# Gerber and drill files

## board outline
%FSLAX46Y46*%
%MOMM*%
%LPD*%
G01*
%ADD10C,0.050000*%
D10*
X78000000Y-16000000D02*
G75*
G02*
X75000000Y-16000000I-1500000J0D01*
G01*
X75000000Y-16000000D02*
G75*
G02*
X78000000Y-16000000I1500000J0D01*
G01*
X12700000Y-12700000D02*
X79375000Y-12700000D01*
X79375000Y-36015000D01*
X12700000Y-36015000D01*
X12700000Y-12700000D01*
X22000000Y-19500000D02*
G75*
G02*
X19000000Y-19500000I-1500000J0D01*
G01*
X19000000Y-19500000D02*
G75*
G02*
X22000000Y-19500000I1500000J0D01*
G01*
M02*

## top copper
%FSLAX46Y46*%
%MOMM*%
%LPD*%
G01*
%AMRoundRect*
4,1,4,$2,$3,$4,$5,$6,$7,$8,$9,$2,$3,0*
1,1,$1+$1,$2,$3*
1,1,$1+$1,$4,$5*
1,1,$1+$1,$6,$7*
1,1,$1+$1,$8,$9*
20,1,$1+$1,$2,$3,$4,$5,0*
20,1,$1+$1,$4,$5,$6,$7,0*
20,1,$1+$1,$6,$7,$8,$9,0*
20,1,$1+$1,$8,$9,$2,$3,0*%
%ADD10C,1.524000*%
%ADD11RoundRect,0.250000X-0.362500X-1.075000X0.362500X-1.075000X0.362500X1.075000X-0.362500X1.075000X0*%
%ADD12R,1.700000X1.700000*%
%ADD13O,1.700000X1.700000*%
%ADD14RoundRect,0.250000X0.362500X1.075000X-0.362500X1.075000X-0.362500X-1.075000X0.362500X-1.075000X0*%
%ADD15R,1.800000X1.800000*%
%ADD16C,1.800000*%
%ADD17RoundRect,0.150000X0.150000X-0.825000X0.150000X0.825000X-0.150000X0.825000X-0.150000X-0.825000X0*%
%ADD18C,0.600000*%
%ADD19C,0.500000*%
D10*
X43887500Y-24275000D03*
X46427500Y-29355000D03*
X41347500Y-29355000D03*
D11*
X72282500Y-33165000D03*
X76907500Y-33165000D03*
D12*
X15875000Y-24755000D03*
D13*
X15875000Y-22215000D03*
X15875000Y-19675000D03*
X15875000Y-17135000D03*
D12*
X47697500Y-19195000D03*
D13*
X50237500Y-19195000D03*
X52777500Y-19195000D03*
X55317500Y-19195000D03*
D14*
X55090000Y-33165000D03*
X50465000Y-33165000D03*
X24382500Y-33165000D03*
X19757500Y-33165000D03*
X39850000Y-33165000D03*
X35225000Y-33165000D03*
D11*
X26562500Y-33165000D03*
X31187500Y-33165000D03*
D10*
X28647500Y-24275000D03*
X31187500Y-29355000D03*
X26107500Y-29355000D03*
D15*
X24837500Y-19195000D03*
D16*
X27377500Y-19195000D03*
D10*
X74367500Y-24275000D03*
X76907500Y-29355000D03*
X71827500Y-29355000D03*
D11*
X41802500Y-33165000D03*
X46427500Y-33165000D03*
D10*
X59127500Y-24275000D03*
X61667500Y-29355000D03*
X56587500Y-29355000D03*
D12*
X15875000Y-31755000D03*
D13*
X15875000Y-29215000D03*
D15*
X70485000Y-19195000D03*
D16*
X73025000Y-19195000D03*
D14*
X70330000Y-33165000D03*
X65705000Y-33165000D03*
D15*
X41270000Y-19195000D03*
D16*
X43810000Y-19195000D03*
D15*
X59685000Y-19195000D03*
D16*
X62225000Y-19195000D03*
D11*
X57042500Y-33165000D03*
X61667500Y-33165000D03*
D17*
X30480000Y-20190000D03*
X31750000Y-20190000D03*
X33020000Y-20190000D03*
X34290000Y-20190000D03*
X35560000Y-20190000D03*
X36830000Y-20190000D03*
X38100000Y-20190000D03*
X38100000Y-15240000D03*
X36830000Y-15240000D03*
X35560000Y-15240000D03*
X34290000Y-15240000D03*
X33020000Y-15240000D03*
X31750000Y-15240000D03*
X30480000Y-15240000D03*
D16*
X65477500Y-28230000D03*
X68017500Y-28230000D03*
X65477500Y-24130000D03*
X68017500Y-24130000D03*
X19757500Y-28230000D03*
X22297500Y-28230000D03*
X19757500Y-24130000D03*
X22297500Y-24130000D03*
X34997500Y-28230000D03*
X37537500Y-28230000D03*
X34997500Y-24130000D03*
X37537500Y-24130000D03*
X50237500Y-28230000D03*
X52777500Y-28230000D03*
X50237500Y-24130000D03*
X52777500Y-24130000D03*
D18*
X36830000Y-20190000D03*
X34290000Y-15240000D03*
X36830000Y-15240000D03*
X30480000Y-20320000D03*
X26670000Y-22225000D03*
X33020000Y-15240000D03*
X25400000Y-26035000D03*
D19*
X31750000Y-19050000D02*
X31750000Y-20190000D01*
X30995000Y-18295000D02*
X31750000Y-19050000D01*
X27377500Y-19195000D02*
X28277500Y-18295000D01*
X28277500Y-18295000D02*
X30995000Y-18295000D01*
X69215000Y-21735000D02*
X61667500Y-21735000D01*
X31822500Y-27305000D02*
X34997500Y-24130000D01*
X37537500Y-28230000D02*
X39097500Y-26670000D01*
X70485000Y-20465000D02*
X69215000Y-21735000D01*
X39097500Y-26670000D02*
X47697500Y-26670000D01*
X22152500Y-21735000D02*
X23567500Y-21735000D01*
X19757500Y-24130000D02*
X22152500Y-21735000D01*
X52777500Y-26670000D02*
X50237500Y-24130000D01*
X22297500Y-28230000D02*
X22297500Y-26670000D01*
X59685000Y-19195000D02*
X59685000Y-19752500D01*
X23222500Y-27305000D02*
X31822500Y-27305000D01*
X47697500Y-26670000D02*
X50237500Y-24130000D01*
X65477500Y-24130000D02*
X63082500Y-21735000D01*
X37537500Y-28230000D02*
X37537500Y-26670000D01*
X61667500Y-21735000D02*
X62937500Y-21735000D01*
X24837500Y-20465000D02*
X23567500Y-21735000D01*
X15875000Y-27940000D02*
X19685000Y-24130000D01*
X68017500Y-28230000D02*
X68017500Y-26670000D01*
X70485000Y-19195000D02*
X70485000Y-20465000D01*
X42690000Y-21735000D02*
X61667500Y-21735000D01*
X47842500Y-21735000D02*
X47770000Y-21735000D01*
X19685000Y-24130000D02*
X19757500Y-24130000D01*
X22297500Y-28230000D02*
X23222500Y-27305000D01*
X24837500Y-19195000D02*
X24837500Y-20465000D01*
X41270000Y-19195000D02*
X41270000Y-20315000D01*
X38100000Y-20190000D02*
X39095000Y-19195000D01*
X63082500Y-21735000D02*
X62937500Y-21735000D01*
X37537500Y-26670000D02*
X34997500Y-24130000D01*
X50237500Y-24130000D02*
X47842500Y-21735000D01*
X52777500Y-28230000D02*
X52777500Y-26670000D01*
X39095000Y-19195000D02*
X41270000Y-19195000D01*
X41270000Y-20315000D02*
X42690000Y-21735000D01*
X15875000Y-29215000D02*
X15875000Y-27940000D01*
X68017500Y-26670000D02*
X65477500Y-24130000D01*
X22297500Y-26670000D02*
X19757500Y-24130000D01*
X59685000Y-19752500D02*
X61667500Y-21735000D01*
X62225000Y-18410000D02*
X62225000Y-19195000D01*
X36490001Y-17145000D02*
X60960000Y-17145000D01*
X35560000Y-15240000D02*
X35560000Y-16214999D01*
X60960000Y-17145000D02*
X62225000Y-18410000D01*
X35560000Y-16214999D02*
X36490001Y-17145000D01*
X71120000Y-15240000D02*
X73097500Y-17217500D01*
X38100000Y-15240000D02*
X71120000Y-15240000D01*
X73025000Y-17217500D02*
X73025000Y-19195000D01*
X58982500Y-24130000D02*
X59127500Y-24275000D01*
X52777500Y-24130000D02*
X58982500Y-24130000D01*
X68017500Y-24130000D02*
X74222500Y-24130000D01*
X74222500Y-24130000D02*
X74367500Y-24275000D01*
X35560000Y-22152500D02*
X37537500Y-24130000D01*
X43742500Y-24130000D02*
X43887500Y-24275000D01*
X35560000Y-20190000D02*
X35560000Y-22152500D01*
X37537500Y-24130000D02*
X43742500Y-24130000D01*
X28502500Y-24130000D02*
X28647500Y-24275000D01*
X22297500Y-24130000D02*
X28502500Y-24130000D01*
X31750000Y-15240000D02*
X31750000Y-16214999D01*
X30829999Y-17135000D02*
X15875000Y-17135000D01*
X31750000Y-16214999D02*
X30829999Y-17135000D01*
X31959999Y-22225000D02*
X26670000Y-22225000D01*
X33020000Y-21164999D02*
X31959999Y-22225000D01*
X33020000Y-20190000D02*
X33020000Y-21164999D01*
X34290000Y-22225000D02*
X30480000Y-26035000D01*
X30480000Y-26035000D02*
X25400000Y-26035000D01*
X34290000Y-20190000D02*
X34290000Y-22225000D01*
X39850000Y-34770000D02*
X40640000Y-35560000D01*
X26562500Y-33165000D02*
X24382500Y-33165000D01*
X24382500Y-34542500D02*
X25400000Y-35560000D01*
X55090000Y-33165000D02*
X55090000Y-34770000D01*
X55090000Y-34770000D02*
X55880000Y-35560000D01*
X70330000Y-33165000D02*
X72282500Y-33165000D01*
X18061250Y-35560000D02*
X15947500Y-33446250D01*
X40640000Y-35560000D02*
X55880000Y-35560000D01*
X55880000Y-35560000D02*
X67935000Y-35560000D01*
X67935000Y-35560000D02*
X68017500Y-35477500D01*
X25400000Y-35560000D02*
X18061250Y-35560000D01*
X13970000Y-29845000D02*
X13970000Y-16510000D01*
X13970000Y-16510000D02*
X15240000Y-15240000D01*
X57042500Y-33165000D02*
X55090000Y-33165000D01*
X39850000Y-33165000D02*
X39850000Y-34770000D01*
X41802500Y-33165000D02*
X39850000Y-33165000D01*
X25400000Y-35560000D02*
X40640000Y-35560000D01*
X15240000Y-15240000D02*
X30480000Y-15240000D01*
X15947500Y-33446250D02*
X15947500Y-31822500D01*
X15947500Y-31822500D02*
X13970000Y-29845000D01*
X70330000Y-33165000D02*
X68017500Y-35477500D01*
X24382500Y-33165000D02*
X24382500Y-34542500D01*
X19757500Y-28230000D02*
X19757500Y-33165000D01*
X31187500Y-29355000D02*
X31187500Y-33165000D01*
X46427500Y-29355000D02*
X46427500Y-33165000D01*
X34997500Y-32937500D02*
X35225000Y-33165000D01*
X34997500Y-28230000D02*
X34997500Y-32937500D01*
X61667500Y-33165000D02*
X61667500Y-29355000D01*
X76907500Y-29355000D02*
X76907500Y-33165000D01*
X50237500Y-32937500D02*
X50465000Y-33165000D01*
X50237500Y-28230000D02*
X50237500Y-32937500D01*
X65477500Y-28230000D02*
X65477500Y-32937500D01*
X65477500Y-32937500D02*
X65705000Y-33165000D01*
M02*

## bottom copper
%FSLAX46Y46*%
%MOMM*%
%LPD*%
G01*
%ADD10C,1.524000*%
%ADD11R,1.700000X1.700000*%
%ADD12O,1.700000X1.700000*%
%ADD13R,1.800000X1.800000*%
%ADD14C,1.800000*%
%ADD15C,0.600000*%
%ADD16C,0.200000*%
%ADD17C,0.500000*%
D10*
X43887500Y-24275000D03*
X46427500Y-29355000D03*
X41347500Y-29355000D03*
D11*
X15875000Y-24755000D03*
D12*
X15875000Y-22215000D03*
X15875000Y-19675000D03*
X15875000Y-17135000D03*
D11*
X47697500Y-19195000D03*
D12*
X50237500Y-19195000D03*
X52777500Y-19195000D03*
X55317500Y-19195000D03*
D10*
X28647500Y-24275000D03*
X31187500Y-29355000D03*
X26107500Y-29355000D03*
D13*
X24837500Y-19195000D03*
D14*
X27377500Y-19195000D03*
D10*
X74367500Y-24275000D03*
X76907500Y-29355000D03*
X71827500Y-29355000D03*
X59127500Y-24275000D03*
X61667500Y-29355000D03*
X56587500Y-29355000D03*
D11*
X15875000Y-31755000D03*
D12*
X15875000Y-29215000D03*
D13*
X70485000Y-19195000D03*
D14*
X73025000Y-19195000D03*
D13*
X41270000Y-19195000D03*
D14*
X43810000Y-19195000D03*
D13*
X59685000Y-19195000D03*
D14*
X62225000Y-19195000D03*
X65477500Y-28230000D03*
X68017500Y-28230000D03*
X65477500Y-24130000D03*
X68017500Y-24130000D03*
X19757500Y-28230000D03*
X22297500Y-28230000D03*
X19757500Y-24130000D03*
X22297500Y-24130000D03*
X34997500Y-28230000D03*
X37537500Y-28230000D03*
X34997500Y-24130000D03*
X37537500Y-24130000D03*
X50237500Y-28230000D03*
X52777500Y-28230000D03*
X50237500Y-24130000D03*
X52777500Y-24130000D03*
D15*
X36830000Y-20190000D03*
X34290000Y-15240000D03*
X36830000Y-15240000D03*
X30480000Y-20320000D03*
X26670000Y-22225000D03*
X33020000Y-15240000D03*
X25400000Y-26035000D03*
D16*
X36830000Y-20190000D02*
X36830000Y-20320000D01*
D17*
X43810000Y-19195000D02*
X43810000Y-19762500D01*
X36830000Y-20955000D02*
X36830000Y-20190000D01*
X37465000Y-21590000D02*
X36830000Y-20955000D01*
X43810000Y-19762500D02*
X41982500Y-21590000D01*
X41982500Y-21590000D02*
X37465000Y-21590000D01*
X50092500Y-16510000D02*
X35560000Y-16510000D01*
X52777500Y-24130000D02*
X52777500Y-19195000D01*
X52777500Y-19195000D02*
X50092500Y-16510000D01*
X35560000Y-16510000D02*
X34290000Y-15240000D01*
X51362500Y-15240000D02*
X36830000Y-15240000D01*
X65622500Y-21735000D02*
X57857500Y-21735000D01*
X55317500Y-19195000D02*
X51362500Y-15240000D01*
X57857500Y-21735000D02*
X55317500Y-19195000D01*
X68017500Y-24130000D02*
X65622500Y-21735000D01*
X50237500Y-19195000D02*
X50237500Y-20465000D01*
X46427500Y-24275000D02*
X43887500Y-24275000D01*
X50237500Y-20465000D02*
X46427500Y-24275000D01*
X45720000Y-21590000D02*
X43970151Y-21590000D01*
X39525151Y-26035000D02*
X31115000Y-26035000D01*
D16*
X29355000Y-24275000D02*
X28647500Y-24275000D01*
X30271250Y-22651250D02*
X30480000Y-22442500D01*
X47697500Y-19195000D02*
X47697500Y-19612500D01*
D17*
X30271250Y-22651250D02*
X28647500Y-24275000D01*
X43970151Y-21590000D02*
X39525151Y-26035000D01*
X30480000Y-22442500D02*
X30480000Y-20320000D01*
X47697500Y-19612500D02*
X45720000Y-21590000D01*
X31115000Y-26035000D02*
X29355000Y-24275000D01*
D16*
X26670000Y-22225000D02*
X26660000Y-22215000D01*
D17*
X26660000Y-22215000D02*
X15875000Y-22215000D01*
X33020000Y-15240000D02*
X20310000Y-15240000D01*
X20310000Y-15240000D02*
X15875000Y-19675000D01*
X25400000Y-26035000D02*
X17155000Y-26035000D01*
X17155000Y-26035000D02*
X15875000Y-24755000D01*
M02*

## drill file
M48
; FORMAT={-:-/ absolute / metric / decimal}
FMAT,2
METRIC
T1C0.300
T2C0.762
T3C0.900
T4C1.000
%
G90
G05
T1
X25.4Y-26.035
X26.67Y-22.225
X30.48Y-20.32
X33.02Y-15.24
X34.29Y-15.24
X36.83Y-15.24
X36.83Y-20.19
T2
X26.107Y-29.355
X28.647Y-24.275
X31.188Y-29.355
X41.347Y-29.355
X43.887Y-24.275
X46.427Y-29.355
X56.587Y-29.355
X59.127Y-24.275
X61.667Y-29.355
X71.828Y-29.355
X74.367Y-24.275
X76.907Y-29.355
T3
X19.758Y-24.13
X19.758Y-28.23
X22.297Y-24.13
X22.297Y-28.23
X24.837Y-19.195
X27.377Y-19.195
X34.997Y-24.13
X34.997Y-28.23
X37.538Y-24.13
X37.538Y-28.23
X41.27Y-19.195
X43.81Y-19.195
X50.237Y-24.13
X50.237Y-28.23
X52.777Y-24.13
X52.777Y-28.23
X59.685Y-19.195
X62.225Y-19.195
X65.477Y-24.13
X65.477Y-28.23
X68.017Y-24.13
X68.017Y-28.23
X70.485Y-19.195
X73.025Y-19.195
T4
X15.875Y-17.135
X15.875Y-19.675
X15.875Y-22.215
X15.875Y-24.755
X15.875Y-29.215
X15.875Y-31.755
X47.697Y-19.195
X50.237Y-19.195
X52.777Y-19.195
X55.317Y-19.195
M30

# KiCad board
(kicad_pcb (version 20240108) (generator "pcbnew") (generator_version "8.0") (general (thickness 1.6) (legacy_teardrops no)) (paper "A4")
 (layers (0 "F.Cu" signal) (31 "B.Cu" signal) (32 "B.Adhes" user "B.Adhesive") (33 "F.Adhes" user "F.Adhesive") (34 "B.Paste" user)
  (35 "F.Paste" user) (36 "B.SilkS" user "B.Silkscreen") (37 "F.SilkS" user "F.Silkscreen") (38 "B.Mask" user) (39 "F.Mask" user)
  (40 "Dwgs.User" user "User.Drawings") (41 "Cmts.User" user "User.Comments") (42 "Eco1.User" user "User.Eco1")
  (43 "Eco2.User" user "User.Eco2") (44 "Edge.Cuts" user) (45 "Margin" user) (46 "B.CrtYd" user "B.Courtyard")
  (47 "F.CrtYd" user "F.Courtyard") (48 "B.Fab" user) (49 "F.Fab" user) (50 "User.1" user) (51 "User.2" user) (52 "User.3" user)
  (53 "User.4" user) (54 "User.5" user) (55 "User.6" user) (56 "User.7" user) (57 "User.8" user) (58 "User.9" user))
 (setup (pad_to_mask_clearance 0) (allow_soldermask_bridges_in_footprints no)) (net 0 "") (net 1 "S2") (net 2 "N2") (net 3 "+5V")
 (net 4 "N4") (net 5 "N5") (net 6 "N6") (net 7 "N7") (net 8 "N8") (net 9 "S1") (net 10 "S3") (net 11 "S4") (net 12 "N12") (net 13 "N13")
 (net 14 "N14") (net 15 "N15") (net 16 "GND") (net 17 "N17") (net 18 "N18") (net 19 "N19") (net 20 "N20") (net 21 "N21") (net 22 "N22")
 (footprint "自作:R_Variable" (layer "F.Cu") (at 43.8875 26.815)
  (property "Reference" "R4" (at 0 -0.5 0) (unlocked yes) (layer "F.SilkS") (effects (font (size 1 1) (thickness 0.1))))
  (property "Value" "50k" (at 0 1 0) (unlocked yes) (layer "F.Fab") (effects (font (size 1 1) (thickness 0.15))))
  (pad "1" thru_hole circle (at 0 -2.54) (size 1.524 1.524) (drill 0.762) (layers "*.Cu" "*.Mask") (remove_unused_layers no) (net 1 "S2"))
  (pad "2" thru_hole circle (at 2.54 2.54) (size 1.524 1.524) (drill 0.762) (layers "*.Cu" "*.Mask") (remove_unused_layers no) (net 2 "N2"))
  (pad "3" thru_hole circle (at -2.54 2.54) (size 1.524 1.524) (drill 0.762) (layers "*.Cu" "*.Mask") (remove_unused_layers no)))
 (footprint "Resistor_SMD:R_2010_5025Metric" (layer "F.Cu") (at 74.595 33.165)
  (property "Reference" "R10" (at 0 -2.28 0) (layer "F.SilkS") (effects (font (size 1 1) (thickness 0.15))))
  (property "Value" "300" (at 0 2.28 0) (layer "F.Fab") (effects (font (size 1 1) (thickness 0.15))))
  (pad "1" smd roundrect (at -2.3125 0) (size 1.225 2.65) (layers "F.Cu" "F.Paste" "F.Mask") (roundrect_rratio 0.204082) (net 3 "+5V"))
  (pad "2" smd roundrect (at 2.3125 0) (size 1.225 2.65) (layers "F.Cu" "F.Paste" "F.Mask") (roundrect_rratio 0.204082) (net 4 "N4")))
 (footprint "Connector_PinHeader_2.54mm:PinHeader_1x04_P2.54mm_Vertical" (layer "F.Cu") (at 15.875 24.755 180)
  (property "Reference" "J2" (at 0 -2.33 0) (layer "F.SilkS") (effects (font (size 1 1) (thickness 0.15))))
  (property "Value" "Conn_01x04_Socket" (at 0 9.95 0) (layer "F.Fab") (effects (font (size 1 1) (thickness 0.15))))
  (pad "1" thru_hole rect (at 0 0 180) (size 1.7 1.7) (drill 1) (layers "*.Cu" "*.Mask") (remove_unused_layers no) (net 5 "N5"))
  (pad "2" thru_hole oval (at 0 2.54 180) (size 1.7 1.7) (drill 1) (layers "*.Cu" "*.Mask") (remove_unused_layers no) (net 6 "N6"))
  (pad "3" thru_hole oval (at 0 5.08 180) (size 1.7 1.7) (drill 1) (layers "*.Cu" "*.Mask") (remove_unused_layers no) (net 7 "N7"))
  (pad "4" thru_hole oval (at 0 7.62 180) (size 1.7 1.7) (drill 1) (layers "*.Cu" "*.Mask") (remove_unused_layers no) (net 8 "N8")))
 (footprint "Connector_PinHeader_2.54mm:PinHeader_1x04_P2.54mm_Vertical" (layer "F.Cu") (at 47.6975 19.195 90)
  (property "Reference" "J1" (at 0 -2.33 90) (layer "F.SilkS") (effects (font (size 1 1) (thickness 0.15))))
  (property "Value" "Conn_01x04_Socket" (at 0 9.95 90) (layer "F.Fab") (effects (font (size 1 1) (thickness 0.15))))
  (pad "1" thru_hole rect (at 0 0 90) (size 1.7 1.7) (drill 1) (layers "*.Cu" "*.Mask") (remove_unused_layers no) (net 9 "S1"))
  (pad "2" thru_hole oval (at 0 2.54 90) (size 1.7 1.7) (drill 1) (layers "*.Cu" "*.Mask") (remove_unused_layers no) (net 1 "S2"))
  (pad "3" thru_hole oval (at 0 5.08 90) (size 1.7 1.7) (drill 1) (layers "*.Cu" "*.Mask") (remove_unused_layers no) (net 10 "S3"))
  (pad "4" thru_hole oval (at 0 7.62 90) (size 1.7 1.7) (drill 1) (layers "*.Cu" "*.Mask") (remove_unused_layers no) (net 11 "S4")))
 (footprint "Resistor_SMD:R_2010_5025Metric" (layer "F.Cu") (at 52.7775 33.165 180)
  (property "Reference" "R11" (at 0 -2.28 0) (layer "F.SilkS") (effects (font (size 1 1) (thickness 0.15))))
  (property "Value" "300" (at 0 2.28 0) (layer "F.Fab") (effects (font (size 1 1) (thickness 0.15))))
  (pad "1" smd roundrect (at -2.3125 0 180) (size 1.225 2.65) (layers "F.Cu" "F.Paste" "F.Mask") (roundrect_rratio 0.204082) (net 3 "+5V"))
  (pad "2" smd roundrect (at 2.3125 0 180) (size 1.225 2.65) (layers "F.Cu" "F.Paste" "F.Mask") (roundrect_rratio 0.204082) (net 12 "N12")))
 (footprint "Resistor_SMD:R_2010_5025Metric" (layer "F.Cu") (at 22.07 33.165 180)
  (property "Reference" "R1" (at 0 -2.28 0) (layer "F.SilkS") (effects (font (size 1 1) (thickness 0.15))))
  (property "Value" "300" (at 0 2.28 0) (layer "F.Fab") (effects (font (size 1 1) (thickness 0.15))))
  (pad "1" smd roundrect (at -2.3125 0 180) (size 1.225 2.65) (layers "F.Cu" "F.Paste" "F.Mask") (roundrect_rratio 0.204082) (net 3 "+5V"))
  (pad "2" smd roundrect (at 2.3125 0 180) (size 1.225 2.65) (layers "F.Cu" "F.Paste" "F.Mask") (roundrect_rratio 0.204082) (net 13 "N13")))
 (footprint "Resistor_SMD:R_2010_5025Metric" (layer "F.Cu") (at 37.5375 33.165 180)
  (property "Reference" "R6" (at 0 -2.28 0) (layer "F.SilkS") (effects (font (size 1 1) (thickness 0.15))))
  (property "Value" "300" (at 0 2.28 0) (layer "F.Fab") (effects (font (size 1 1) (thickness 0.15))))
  (pad "1" smd roundrect (at -2.3125 0 180) (size 1.225 2.65) (layers "F.Cu" "F.Paste" "F.Mask") (roundrect_rratio 0.204082) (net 3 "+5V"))
  (pad "2" smd roundrect (at 2.3125 0 180) (size 1.225 2.65) (layers "F.Cu" "F.Paste" "F.Mask") (roundrect_rratio 0.204082) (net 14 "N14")))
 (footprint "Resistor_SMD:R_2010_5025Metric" (layer "F.Cu") (at 28.875 33.165)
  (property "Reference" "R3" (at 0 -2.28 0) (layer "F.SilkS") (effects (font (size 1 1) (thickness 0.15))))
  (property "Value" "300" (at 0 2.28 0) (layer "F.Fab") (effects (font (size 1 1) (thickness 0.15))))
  (pad "1" smd roundrect (at -2.3125 0) (size 1.225 2.65) (layers "F.Cu" "F.Paste" "F.Mask") (roundrect_rratio 0.204082) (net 3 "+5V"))
  (pad "2" smd roundrect (at 2.3125 0) (size 1.225 2.65) (layers "F.Cu" "F.Paste" "F.Mask") (roundrect_rratio 0.204082) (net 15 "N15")))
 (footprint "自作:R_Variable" (layer "F.Cu") (at 28.6475 26.815)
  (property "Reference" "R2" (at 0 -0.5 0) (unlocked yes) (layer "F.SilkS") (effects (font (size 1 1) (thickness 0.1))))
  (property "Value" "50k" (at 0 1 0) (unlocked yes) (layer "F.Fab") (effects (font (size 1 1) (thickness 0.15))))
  (pad "1" thru_hole circle (at 0 -2.54) (size 1.524 1.524) (drill 0.762) (layers "*.Cu" "*.Mask") (remove_unused_layers no) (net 9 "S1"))
  (pad "2" thru_hole circle (at 2.54 2.54) (size 1.524 1.524) (drill 0.762) (layers "*.Cu" "*.Mask") (remove_unused_layers no)
   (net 15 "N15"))
  (pad "3" thru_hole circle (at -2.54 2.54) (size 1.524 1.524) (drill 0.762) (layers "*.Cu" "*.Mask") (remove_unused_layers no)))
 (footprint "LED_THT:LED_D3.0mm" (layer "F.Cu") (at 24.8375 19.195)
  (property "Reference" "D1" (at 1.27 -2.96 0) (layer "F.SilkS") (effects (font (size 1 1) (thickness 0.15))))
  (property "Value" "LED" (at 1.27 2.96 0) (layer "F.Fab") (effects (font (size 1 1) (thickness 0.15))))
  (pad "1" thru_hole rect (at 0 0) (size 1.8 1.8) (drill 0.9) (layers "*.Cu" "*.Mask") (remove_unused_layers no) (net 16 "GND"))
  (pad "2" thru_hole circle (at 2.54 0) (size 1.8 1.8) (drill 0.9) (layers "*.Cu" "*.Mask") (remove_unused_layers no) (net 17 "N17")))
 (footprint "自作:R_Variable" (layer "F.Cu") (at 74.3675 26.815)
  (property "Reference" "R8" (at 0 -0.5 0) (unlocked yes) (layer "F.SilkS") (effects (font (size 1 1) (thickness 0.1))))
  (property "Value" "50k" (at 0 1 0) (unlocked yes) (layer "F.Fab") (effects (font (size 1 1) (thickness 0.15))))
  (pad "1" thru_hole circle (at 0 -2.54) (size 1.524 1.524) (drill 0.762) (layers "*.Cu" "*.Mask") (remove_unused_layers no) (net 11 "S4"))
  (pad "2" thru_hole circle (at 2.54 2.54) (size 1.524 1.524) (drill 0.762) (layers "*.Cu" "*.Mask") (remove_unused_layers no) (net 4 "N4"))
  (pad "3" thru_hole circle (at -2.54 2.54) (size 1.524 1.524) (drill 0.762) (layers "*.Cu" "*.Mask") (remove_unused_layers no)))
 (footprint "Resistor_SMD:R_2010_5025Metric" (layer "F.Cu") (at 44.115 33.165)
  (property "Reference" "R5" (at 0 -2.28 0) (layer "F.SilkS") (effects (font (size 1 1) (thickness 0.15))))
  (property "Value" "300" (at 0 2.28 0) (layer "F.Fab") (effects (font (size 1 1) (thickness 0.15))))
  (pad "1" smd roundrect (at -2.3125 0) (size 1.225 2.65) (layers "F.Cu" "F.Paste" "F.Mask") (roundrect_rratio 0.204082) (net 3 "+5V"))
  (pad "2" smd roundrect (at 2.3125 0) (size 1.225 2.65) (layers "F.Cu" "F.Paste" "F.Mask") (roundrect_rratio 0.204082) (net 2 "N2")))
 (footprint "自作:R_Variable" (layer "F.Cu") (at 59.1275 26.815)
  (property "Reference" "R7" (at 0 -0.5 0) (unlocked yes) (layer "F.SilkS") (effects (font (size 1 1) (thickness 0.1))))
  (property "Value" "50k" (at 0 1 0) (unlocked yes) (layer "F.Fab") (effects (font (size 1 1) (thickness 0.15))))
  (pad "1" thru_hole circle (at 0 -2.54) (size 1.524 1.524) (drill 0.762) (layers "*.Cu" "*.Mask") (remove_unused_layers no) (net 10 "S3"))
  (pad "2" thru_hole circle (at 2.54 2.54) (size 1.524 1.524) (drill 0.762) (layers "*.Cu" "*.Mask") (remove_unused_layers no)
   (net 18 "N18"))
  (pad "3" thru_hole circle (at -2.54 2.54) (size 1.524 1.524) (drill 0.762) (layers "*.Cu" "*.Mask") (remove_unused_layers no)))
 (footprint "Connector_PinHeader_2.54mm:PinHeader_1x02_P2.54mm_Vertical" (layer "F.Cu") (at 15.875 31.755 180)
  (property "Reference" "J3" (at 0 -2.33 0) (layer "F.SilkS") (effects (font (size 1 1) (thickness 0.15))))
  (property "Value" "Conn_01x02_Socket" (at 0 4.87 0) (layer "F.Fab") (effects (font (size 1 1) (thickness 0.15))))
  (pad "1" thru_hole rect (at 0 0 180) (size 1.7 1.7) (drill 1) (layers "*.Cu" "*.Mask") (remove_unused_layers no) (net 3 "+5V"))
  (pad "2" thru_hole oval (at 0 2.54 180) (size 1.7 1.7) (drill 1) (layers "*.Cu" "*.Mask") (remove_unused_layers no) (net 16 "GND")))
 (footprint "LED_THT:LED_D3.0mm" (layer "F.Cu") (at 70.485 19.195)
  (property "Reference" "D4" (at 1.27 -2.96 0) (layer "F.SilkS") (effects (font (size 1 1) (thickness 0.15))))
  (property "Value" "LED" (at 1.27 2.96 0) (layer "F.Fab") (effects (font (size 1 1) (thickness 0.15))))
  (pad "1" thru_hole rect (at 0 0) (size 1.8 1.8) (drill 0.9) (layers "*.Cu" "*.Mask") (remove_unused_layers no) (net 16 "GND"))
  (pad "2" thru_hole circle (at 2.54 0) (size 1.8 1.8) (drill 0.9) (layers "*.Cu" "*.Mask") (remove_unused_layers no) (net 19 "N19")))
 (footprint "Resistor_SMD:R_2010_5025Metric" (layer "F.Cu") (at 68.0175 33.165 180)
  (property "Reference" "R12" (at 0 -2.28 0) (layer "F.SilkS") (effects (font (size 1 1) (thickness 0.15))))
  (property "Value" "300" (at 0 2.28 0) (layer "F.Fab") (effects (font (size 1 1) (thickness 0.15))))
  (pad "1" smd roundrect (at -2.3125 0 180) (size 1.225 2.65) (layers "F.Cu" "F.Paste" "F.Mask") (roundrect_rratio 0.204082) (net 3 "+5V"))
  (pad "2" smd roundrect (at 2.3125 0 180) (size 1.225 2.65) (layers "F.Cu" "F.Paste" "F.Mask") (roundrect_rratio 0.204082) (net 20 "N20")))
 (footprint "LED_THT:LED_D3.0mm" (layer "F.Cu") (at 41.27 19.195)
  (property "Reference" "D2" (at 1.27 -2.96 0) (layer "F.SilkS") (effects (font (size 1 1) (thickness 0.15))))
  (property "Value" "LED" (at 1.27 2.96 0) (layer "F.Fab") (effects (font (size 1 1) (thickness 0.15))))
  (pad "1" thru_hole rect (at 0 0) (size 1.8 1.8) (drill 0.9) (layers "*.Cu" "*.Mask") (remove_unused_layers no) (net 16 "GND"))
  (pad "2" thru_hole circle (at 2.54 0) (size 1.8 1.8) (drill 0.9) (layers "*.Cu" "*.Mask") (remove_unused_layers no) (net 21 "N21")))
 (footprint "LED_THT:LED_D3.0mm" (layer "F.Cu") (at 59.685 19.195)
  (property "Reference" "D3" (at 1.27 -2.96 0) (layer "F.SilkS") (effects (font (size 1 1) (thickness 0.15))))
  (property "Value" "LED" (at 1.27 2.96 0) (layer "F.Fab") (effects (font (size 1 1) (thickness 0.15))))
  (pad "1" thru_hole rect (at 0 0) (size 1.8 1.8) (drill 0.9) (layers "*.Cu" "*.Mask") (remove_unused_layers no) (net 16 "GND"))
  (pad "2" thru_hole circle (at 2.54 0) (size 1.8 1.8) (drill 0.9) (layers "*.Cu" "*.Mask") (remove_unused_layers no) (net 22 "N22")))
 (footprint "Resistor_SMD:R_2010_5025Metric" (layer "F.Cu") (at 59.355 33.165)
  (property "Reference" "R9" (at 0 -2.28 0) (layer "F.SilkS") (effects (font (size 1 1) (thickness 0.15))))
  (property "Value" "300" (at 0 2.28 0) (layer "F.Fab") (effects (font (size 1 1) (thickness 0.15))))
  (pad "1" smd roundrect (at -2.3125 0) (size 1.225 2.65) (layers "F.Cu" "F.Paste" "F.Mask") (roundrect_rratio 0.204082) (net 3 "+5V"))
  (pad "2" smd roundrect (at 2.3125 0) (size 1.225 2.65) (layers "F.Cu" "F.Paste" "F.Mask") (roundrect_rratio 0.204082) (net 18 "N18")))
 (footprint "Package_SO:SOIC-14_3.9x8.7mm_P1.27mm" (layer "F.Cu") (at 34.29 17.715 90)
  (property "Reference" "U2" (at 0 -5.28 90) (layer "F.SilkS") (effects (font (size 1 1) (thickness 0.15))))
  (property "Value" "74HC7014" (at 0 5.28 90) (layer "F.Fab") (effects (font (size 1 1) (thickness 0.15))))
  (pad "1" smd roundrect (at -2.475 -3.81 90) (size 1.95 0.6) (layers "F.Cu" "F.Paste" "F.Mask") (roundrect_rratio 0.25) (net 9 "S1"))
  (pad "2" smd roundrect (at -2.475 -2.54 90) (size 1.95 0.6) (layers "F.Cu" "F.Paste" "F.Mask") (roundrect_rratio 0.25) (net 17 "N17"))
  (pad "3" smd roundrect (at -2.475 -1.27 90) (size 1.95 0.6) (layers "F.Cu" "F.Paste" "F.Mask") (roundrect_rratio 0.25) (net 6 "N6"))
  (pad "4" smd roundrect (at -2.475 0 90) (size 1.95 0.6) (layers "F.Cu" "F.Paste" "F.Mask") (roundrect_rratio 0.25) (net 5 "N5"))
  (pad "5" smd roundrect (at -2.475 1.27 90) (size 1.95 0.6) (layers "F.Cu" "F.Paste" "F.Mask") (roundrect_rratio 0.25) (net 1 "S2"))
  (pad "6" smd roundrect (at -2.475 2.54 90) (size 1.95 0.6) (layers "F.Cu" "F.Paste" "F.Mask") (roundrect_rratio 0.25) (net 21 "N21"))
  (pad "7" smd roundrect (at -2.475 3.81 90) (size 1.95 0.6) (layers "F.Cu" "F.Paste" "F.Mask") (roundrect_rratio 0.25) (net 16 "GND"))
  (pad "8" smd roundrect (at 2.475 3.81 90) (size 1.95 0.6) (layers "F.Cu" "F.Paste" "F.Mask") (roundrect_rratio 0.25) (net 19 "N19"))
  (pad "9" smd roundrect (at 2.475 2.54 90) (size 1.95 0.6) (layers "F.Cu" "F.Paste" "F.Mask") (roundrect_rratio 0.25) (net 11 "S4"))
  (pad "10" smd roundrect (at 2.475 1.27 90) (size 1.95 0.6) (layers "F.Cu" "F.Paste" "F.Mask") (roundrect_rratio 0.25) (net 22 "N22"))
  (pad "11" smd roundrect (at 2.475 0 90) (size 1.95 0.6) (layers "F.Cu" "F.Paste" "F.Mask") (roundrect_rratio 0.25) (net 10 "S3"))
  (pad "12" smd roundrect (at 2.475 -1.27 90) (size 1.95 0.6) (layers "F.Cu" "F.Paste" "F.Mask") (roundrect_rratio 0.25) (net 7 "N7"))
  (pad "13" smd roundrect (at 2.475 -2.54 90) (size 1.95 0.6) (layers "F.Cu" "F.Paste" "F.Mask") (roundrect_rratio 0.25) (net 8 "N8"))
  (pad "14" smd roundrect (at 2.475 -3.81 90) (size 1.95 0.6) (layers "F.Cu" "F.Paste" "F.Mask") (roundrect_rratio 0.25) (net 3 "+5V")))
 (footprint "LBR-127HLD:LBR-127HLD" (layer "B.Cu") (at 66.7475 26.18 -90)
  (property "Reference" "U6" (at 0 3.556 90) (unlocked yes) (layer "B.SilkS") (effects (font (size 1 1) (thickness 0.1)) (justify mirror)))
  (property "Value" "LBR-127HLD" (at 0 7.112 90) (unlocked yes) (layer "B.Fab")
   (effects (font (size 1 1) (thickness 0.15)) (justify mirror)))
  (pad "1" thru_hole circle (at 2.05 1.27 270) (size 1.8 1.8) (drill 0.9) (layers "*.Cu" "*.Mask") (remove_unused_layers no) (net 20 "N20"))
  (pad "2" thru_hole circle (at 2.05 -1.27 270) (size 1.8 1.8) (drill 0.9) (layers "*.Cu" "*.Mask") (remove_unused_layers no) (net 16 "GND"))
  (pad "3" thru_hole circle (at -2.05 1.27 270) (size 1.8 1.8) (drill 0.9) (layers "*.Cu" "*.Mask") (remove_unused_layers no) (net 16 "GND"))
  (pad "4" thru_hole circle (at -2.05 -1.27 270) (size 1.8 1.8) (drill 0.9) (layers "*.Cu" "*.Mask") (remove_unused_layers no) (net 11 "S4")))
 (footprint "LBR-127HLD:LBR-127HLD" (layer "B.Cu") (at 21.0275 26.18 -90)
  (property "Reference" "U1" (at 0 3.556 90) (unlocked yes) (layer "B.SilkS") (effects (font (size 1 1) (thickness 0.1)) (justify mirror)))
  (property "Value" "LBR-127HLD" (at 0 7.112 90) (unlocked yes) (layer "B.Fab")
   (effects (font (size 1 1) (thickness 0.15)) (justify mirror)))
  (pad "1" thru_hole circle (at 2.05 1.27 270) (size 1.8 1.8) (drill 0.9) (layers "*.Cu" "*.Mask") (remove_unused_layers no) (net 13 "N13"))
  (pad "2" thru_hole circle (at 2.05 -1.27 270) (size 1.8 1.8) (drill 0.9) (layers "*.Cu" "*.Mask") (remove_unused_layers no) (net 16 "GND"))
  (pad "3" thru_hole circle (at -2.05 1.27 270) (size 1.8 1.8) (drill 0.9) (layers "*.Cu" "*.Mask") (remove_unused_layers no) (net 16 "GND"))
  (pad "4" thru_hole circle (at -2.05 -1.27 270) (size 1.8 1.8) (drill 0.9) (layers "*.Cu" "*.Mask") (remove_unused_layers no) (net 9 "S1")))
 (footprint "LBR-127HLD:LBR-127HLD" (layer "B.Cu") (at 36.2675 26.18 -90)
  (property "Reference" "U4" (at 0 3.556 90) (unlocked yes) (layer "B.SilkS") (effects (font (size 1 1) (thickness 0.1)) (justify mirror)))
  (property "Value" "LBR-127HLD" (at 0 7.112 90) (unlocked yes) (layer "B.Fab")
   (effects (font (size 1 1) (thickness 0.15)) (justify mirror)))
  (pad "1" thru_hole circle (at 2.05 1.27 270) (size 1.8 1.8) (drill 0.9) (layers "*.Cu" "*.Mask") (remove_unused_layers no) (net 14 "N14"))
  (pad "2" thru_hole circle (at 2.05 -1.27 270) (size 1.8 1.8) (drill 0.9) (layers "*.Cu" "*.Mask") (remove_unused_layers no) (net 16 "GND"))
  (pad "3" thru_hole circle (at -2.05 1.27 270) (size 1.8 1.8) (drill 0.9) (layers "*.Cu" "*.Mask") (remove_unused_layers no) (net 16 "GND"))
  (pad "4" thru_hole circle (at -2.05 -1.27 270) (size 1.8 1.8) (drill 0.9) (layers "*.Cu" "*.Mask") (remove_unused_layers no) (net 1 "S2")))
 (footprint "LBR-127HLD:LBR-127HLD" (layer "B.Cu") (at 51.5075 26.18 -90)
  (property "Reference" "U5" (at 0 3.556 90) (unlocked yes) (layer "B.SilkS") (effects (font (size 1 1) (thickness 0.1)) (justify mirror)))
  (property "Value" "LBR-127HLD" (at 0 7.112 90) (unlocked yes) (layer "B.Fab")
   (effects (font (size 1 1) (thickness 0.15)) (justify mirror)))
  (pad "1" thru_hole circle (at 2.05 1.27 270) (size 1.8 1.8) (drill 0.9) (layers "*.Cu" "*.Mask") (remove_unused_layers no) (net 12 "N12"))
  (pad "2" thru_hole circle (at 2.05 -1.27 270) (size 1.8 1.8) (drill 0.9) (layers "*.Cu" "*.Mask") (remove_unused_layers no) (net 16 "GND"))
  (pad "3" thru_hole circle (at -2.05 1.27 270) (size 1.8 1.8) (drill 0.9) (layers "*.Cu" "*.Mask") (remove_unused_layers no) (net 16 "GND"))
  (pad "4" thru_hole circle (at -2.05 -1.27 270) (size 1.8 1.8) (drill 0.9) (layers "*.Cu" "*.Mask") (remove_unused_layers no) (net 10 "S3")))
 (gr_circle (center 76.5 16) (end 78 16) (stroke (width 0.05) (type default)) (fill none) (layer "Edge.Cuts"))
 (gr_rect (start 12.7 12.7) (end 79.375 36.015) (stroke (width 0.05) (type default)) (fill none) (layer "Edge.Cuts"))
 (gr_circle (center 20.5 19.5) (end 22 19.5) (stroke (width 0.05) (type default)) (fill none) (layer "Edge.Cuts"))
 (segment (start 31.75 19.05) (end 31.75 20.19) (width 0.5) (layer "F.Cu") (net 17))
 (segment (start 30.995 18.295) (end 31.75 19.05) (width 0.5) (layer "F.Cu") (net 17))
 (segment (start 27.3775 19.195) (end 28.2775 18.295) (width 0.5) (layer "F.Cu") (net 17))
 (segment (start 28.2775 18.295) (end 30.995 18.295) (width 0.5) (layer "F.Cu") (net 17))
 (segment (start 69.215 21.735) (end 61.6675 21.735) (width 0.5) (layer "F.Cu") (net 16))
 (segment (start 31.8225 27.305) (end 34.9975 24.13) (width 0.5) (layer "F.Cu") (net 16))
 (segment (start 37.5375 28.23) (end 39.0975 26.67) (width 0.5) (layer "F.Cu") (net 16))
 (segment (start 70.485 20.465) (end 69.215 21.735) (width 0.5) (layer "F.Cu") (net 16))
 (segment (start 39.0975 26.67) (end 47.6975 26.67) (width 0.5) (layer "F.Cu") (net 16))
 (segment (start 22.1525 21.735) (end 23.5675 21.735) (width 0.5) (layer "F.Cu") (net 16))
 (segment (start 19.7575 24.13) (end 22.1525 21.735) (width 0.5) (layer "F.Cu") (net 16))
 (segment (start 52.7775 26.67) (end 50.2375 24.13) (width 0.5) (layer "F.Cu") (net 16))
 (segment (start 22.2975 28.23) (end 22.2975 26.67) (width 0.5) (layer "F.Cu") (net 16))
 (segment (start 59.685 19.195) (end 59.685 19.7525) (width 0.5) (layer "F.Cu") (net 16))
 (segment (start 23.2225 27.305) (end 31.8225 27.305) (width 0.5) (layer "F.Cu") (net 16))
 (segment (start 47.6975 26.67) (end 50.2375 24.13) (width 0.5) (layer "F.Cu") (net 16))
 (segment (start 65.4775 24.13) (end 63.0825 21.735) (width 0.5) (layer "F.Cu") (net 16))
 (segment (start 37.5375 28.23) (end 37.5375 26.67) (width 0.5) (layer "F.Cu") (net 16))
 (segment (start 61.6675 21.735) (end 62.9375 21.735) (width 0.5) (layer "F.Cu") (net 16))
 (segment (start 24.8375 20.465) (end 23.5675 21.735) (width 0.5) (layer "F.Cu") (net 16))
 (segment (start 15.875 27.94) (end 19.685 24.13) (width 0.5) (layer "F.Cu") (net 16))
 (segment (start 68.0175 28.23) (end 68.0175 26.67) (width 0.5) (layer "F.Cu") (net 16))
 (segment (start 70.485 19.195) (end 70.485 20.465) (width 0.5) (layer "F.Cu") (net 16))
 (segment (start 42.69 21.735) (end 61.6675 21.735) (width 0.5) (layer "F.Cu") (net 16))
 (segment (start 47.8425 21.735) (end 47.77 21.735) (width 0.5) (layer "F.Cu") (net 16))
 (segment (start 19.685 24.13) (end 19.7575 24.13) (width 0.5) (layer "F.Cu") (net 16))
 (segment (start 22.2975 28.23) (end 23.2225 27.305) (width 0.5) (layer "F.Cu") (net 16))
 (segment (start 24.8375 19.195) (end 24.8375 20.465) (width 0.5) (layer "F.Cu") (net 16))
 (segment (start 41.27 19.195) (end 41.27 20.315) (width 0.5) (layer "F.Cu") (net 16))
 (segment (start 38.1 20.19) (end 39.095 19.195) (width 0.5) (layer "F.Cu") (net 16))
 (segment (start 63.0825 21.735) (end 62.9375 21.735) (width 0.5) (layer "F.Cu") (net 16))
 (segment (start 37.5375 26.67) (end 34.9975 24.13) (width 0.5) (layer "F.Cu") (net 16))
 (segment (start 50.2375 24.13) (end 47.8425 21.735) (width 0.5) (layer "F.Cu") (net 16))
 (segment (start 52.7775 28.23) (end 52.7775 26.67) (width 0.5) (layer "F.Cu") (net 16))
 (segment (start 39.095 19.195) (end 41.27 19.195) (width 0.5) (layer "F.Cu") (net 16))
 (segment (start 41.27 20.315) (end 42.69 21.735) (width 0.5) (layer "F.Cu") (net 16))
 (segment (start 15.875 29.215) (end 15.875 27.94) (width 0.5) (layer "F.Cu") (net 16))
 (segment (start 68.0175 26.67) (end 65.4775 24.13) (width 0.5) (layer "F.Cu") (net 16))
 (segment (start 22.2975 26.67) (end 19.7575 24.13) (width 0.5) (layer "F.Cu") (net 16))
 (segment (start 59.685 19.7525) (end 61.6675 21.735) (width 0.5) (layer "F.Cu") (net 16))
 (via (at 36.83 20.19) (size 0.6) (drill 0.3) (layers "F.Cu" "B.Cu") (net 21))
 (segment (start 36.83 20.19) (end 36.83 20.32) (width 0.2) (layer "B.Cu") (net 21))
 (segment (start 43.81 19.195) (end 43.81 19.7625) (width 0.5) (layer "B.Cu") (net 21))
 (segment (start 36.83 20.955) (end 36.83 20.19) (width 0.5) (layer "B.Cu") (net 21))
 (segment (start 37.465 21.59) (end 36.83 20.955) (width 0.5) (layer "B.Cu") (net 21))
 (segment (start 43.81 19.7625) (end 41.9825 21.59) (width 0.5) (layer "B.Cu") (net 21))
 (segment (start 41.9825 21.59) (end 37.465 21.59) (width 0.5) (layer "B.Cu") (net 21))
 (segment (start 62.225 18.41) (end 62.225 19.195) (width 0.5) (layer "F.Cu") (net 22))
 (segment (start 36.490001 17.145) (end 60.96 17.145) (width 0.5) (layer "F.Cu") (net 22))
 (segment (start 35.56 15.24) (end 35.56 16.214999) (width 0.5) (layer "F.Cu") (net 22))
 (segment (start 60.96 17.145) (end 62.225 18.41) (width 0.5) (layer "F.Cu") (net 22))
 (segment (start 35.56 16.214999) (end 36.490001 17.145) (width 0.5) (layer "F.Cu") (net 22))
 (segment (start 71.12 15.24) (end 73.0975 17.2175) (width 0.5) (layer "F.Cu") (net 19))
 (segment (start 38.1 15.24) (end 71.12 15.24) (width 0.5) (layer "F.Cu") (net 19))
 (segment (start 73.025 17.2175) (end 73.025 19.195) (width 0.5) (layer "F.Cu") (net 19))
 (segment (start 58.9825 24.13) (end 59.1275 24.275) (width 0.5) (layer "F.Cu") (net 10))
 (segment (start 52.7775 24.13) (end 58.9825 24.13) (width 0.5) (layer "F.Cu") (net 10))
 (via (at 34.29 15.24) (size 0.6) (drill 0.3) (layers "F.Cu" "B.Cu") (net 10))
 (segment (start 50.0925 16.51) (end 35.56 16.51) (width 0.5) (layer "B.Cu") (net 10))
 (segment (start 52.7775 24.13) (end 52.7775 19.195) (width 0.5) (layer "B.Cu") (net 10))
 (segment (start 52.7775 19.195) (end 50.0925 16.51) (width 0.5) (layer "B.Cu") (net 10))
 (segment (start 35.56 16.51) (end 34.29 15.24) (width 0.5) (layer "B.Cu") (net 10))
 (segment (start 68.0175 24.13) (end 74.2225 24.13) (width 0.5) (layer "F.Cu") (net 11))
 (segment (start 74.2225 24.13) (end 74.3675 24.275) (width 0.5) (layer "F.Cu") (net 11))
 (via (at 36.83 15.24) (size 0.6) (drill 0.3) (layers "F.Cu" "B.Cu") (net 11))
 (segment (start 51.3625 15.24) (end 36.83 15.24) (width 0.5) (layer "B.Cu") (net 11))
 (segment (start 65.6225 21.735) (end 57.8575 21.735) (width 0.5) (layer "B.Cu") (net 11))
 (segment (start 55.3175 19.195) (end 51.3625 15.24) (width 0.5) (layer "B.Cu") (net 11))
 (segment (start 57.8575 21.735) (end 55.3175 19.195) (width 0.5) (layer "B.Cu") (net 11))
 (segment (start 68.0175 24.13) (end 65.6225 21.735) (width 0.5) (layer "B.Cu") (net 11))
 (segment (start 35.56 22.1525) (end 37.5375 24.13) (width 0.5) (layer "F.Cu") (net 1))
 (segment (start 43.7425 24.13) (end 43.8875 24.275) (width 0.5) (layer "F.Cu") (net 1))
 (segment (start 35.56 20.19) (end 35.56 22.1525) (width 0.5) (layer "F.Cu") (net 1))
 (segment (start 37.5375 24.13) (end 43.7425 24.13) (width 0.5) (layer "F.Cu") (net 1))
 (segment (start 50.2375 19.195) (end 50.2375 20.465) (width 0.5) (layer "B.Cu") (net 1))
 (segment (start 46.4275 24.275) (end 43.8875 24.275) (width 0.5) (layer "B.Cu") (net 1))
 (segment (start 50.2375 20.465) (end 46.4275 24.275) (width 0.5) (layer "B.Cu") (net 1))
 (segment (start 28.5025 24.13) (end 28.6475 24.275) (width 0.5) (layer "F.Cu") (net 9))
 (segment (start 22.2975 24.13) (end 28.5025 24.13) (width 0.5) (layer "F.Cu") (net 9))
 (via (at 30.48 20.32) (size 0.6) (drill 0.3) (layers "F.Cu" "B.Cu") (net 9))
 (segment (start 45.72 21.59) (end 43.970151 21.59) (width 0.5) (layer "B.Cu") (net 9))
 (segment (start 39.525151 26.035) (end 31.115 26.035) (width 0.5) (layer "B.Cu") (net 9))
 (segment (start 29.355 24.275) (end 28.6475 24.275) (width 0.2) (layer "B.Cu") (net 9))
 (segment (start 30.27125 22.65125) (end 30.48 22.4425) (width 0.2) (layer "B.Cu") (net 9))
 (segment (start 47.6975 19.195) (end 47.6975 19.6125) (width 0.2) (layer "B.Cu") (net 9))
 (segment (start 30.27125 22.65125) (end 28.6475 24.275) (width 0.5) (layer "B.Cu") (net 9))
 (segment (start 43.970151 21.59) (end 39.525151 26.035) (width 0.5) (layer "B.Cu") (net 9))
 (segment (start 30.48 22.4425) (end 30.48 20.32) (width 0.5) (layer "B.Cu") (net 9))
 (segment (start 47.6975 19.6125) (end 45.72 21.59) (width 0.5) (layer "B.Cu") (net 9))
 (segment (start 31.115 26.035) (end 29.355 24.275) (width 0.5) (layer "B.Cu") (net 9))
 (segment (start 31.75 15.24) (end 31.75 16.214999) (width 0.5) (layer "F.Cu") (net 8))
 (segment (start 30.829999 17.135) (end 15.875 17.135) (width 0.5) (layer "F.Cu") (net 8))
 (segment (start 31.75 16.214999) (end 30.829999 17.135) (width 0.5) (layer "F.Cu") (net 8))
 (segment (start 31.959999 22.225) (end 26.67 22.225) (width 0.5) (layer "F.Cu") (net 6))
 (segment (start 33.02 21.164999) (end 31.959999 22.225) (width 0.5) (layer "F.Cu") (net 6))
 (segment (start 33.02 20.19) (end 33.02 21.164999) (width 0.5) (layer "F.Cu") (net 6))
 (via (at 26.67 22.225) (size 0.6) (drill 0.3) (layers "F.Cu" "B.Cu") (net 6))
 (segment (start 26.67 22.225) (end 26.66 22.215) (width 0.2) (layer "B.Cu") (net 6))
 (segment (start 26.66 22.215) (end 15.875 22.215) (width 0.5) (layer "B.Cu") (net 6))
 (via (at 33.02 15.24) (size 0.6) (drill 0.3) (layers "F.Cu" "B.Cu") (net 7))
 (segment (start 33.02 15.24) (end 20.31 15.24) (width 0.5) (layer "B.Cu") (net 7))
 (segment (start 20.31 15.24) (end 15.875 19.675) (width 0.5) (layer "B.Cu") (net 7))
 (segment (start 34.29 22.225) (end 30.48 26.035) (width 0.5) (layer "F.Cu") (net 5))
 (segment (start 30.48 26.035) (end 25.4 26.035) (width 0.5) (layer "F.Cu") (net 5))
 (segment (start 34.29 20.19) (end 34.29 22.225) (width 0.5) (layer "F.Cu") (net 5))
 (via (at 25.4 26.035) (size 0.6) (drill 0.3) (layers "F.Cu" "B.Cu") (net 5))
 (segment (start 25.4 26.035) (end 17.155 26.035) (width 0.5) (layer "B.Cu") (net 5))
 (segment (start 17.155 26.035) (end 15.875 24.755) (width 0.5) (layer "B.Cu") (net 5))
 (segment (start 39.85 34.77) (end 40.64 35.56) (width 0.5) (layer "F.Cu") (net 3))
 (segment (start 26.5625 33.165) (end 24.3825 33.165) (width 0.5) (layer "F.Cu") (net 3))
 (segment (start 24.3825 34.5425) (end 25.4 35.56) (width 0.5) (layer "F.Cu") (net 3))
 (segment (start 55.09 33.165) (end 55.09 34.77) (width 0.5) (layer "F.Cu") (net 3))
 (segment (start 55.09 34.77) (end 55.88 35.56) (width 0.5) (layer "F.Cu") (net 3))
 (segment (start 70.33 33.165) (end 72.2825 33.165) (width 0.5) (layer "F.Cu") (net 3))
 (segment (start 18.06125 35.56) (end 15.9475 33.44625) (width 0.5) (layer "F.Cu") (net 3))
 (segment (start 40.64 35.56) (end 55.88 35.56) (width 0.5) (layer "F.Cu") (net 3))
 (segment (start 55.88 35.56) (end 67.935 35.56) (width 0.5) (layer "F.Cu") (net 3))
 (segment (start 67.935 35.56) (end 68.0175 35.4775) (width 0.5) (layer "F.Cu") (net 3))
 (segment (start 25.4 35.56) (end 18.06125 35.56) (width 0.5) (layer "F.Cu") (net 3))
 (segment (start 13.97 29.845) (end 13.97 16.51) (width 0.5) (layer "F.Cu") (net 3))
 (segment (start 13.97 16.51) (end 15.24 15.24) (width 0.5) (layer "F.Cu") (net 3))
 (segment (start 57.0425 33.165) (end 55.09 33.165) (width 0.5) (layer "F.Cu") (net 3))
 (segment (start 39.85 33.165) (end 39.85 34.77) (width 0.5) (layer "F.Cu") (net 3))
 (segment (start 41.8025 33.165) (end 39.85 33.165) (width 0.5) (layer "F.Cu") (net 3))
 (segment (start 25.4 35.56) (end 40.64 35.56) (width 0.5) (layer "F.Cu") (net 3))
 (segment (start 15.24 15.24) (end 30.48 15.24) (width 0.5) (layer "F.Cu") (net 3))
 (segment (start 15.9475 33.44625) (end 15.9475 31.8225) (width 0.5) (layer "F.Cu") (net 3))
 (segment (start 15.9475 31.8225) (end 13.97 29.845) (width 0.5) (layer "F.Cu") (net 3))
 (segment (start 70.33 33.165) (end 68.0175 35.4775) (width 0.5) (layer "F.Cu") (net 3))
 (segment (start 24.3825 33.165) (end 24.3825 34.5425) (width 0.5) (layer "F.Cu") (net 3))
 (segment (start 19.7575 28.23) (end 19.7575 33.165) (width 0.5) (layer "F.Cu") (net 13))
 (segment (start 31.1875 29.355) (end 31.1875 33.165) (width 0.5) (layer "F.Cu") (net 15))
 (segment (start 46.4275 29.355) (end 46.4275 33.165) (width 0.5) (layer "F.Cu") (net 2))
 (segment (start 34.9975 32.9375) (end 35.225 33.165) (width 0.5) (layer "F.Cu") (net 14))
 (segment (start 34.9975 28.23) (end 34.9975 32.9375) (width 0.5) (layer "F.Cu") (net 14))
 (segment (start 61.6675 33.165) (end 61.6675 29.355) (width 0.5) (layer "F.Cu") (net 18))
 (segment (start 76.9075 29.355) (end 76.9075 33.165) (width 0.5) (layer "F.Cu") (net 4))
 (segment (start 50.2375 32.9375) (end 50.465 33.165) (width 0.5) (layer "F.Cu") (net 12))
 (segment (start 50.2375 28.23) (end 50.2375 32.9375) (width 0.5) (layer "F.Cu") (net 12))
 (segment (start 65.4775 28.23) (end 65.4775 32.9375) (width 0.5) (layer "F.Cu") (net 20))
 (segment (start 65.4775 32.9375) (end 65.705 33.165) (width 0.5) (layer "F.Cu") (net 20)))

